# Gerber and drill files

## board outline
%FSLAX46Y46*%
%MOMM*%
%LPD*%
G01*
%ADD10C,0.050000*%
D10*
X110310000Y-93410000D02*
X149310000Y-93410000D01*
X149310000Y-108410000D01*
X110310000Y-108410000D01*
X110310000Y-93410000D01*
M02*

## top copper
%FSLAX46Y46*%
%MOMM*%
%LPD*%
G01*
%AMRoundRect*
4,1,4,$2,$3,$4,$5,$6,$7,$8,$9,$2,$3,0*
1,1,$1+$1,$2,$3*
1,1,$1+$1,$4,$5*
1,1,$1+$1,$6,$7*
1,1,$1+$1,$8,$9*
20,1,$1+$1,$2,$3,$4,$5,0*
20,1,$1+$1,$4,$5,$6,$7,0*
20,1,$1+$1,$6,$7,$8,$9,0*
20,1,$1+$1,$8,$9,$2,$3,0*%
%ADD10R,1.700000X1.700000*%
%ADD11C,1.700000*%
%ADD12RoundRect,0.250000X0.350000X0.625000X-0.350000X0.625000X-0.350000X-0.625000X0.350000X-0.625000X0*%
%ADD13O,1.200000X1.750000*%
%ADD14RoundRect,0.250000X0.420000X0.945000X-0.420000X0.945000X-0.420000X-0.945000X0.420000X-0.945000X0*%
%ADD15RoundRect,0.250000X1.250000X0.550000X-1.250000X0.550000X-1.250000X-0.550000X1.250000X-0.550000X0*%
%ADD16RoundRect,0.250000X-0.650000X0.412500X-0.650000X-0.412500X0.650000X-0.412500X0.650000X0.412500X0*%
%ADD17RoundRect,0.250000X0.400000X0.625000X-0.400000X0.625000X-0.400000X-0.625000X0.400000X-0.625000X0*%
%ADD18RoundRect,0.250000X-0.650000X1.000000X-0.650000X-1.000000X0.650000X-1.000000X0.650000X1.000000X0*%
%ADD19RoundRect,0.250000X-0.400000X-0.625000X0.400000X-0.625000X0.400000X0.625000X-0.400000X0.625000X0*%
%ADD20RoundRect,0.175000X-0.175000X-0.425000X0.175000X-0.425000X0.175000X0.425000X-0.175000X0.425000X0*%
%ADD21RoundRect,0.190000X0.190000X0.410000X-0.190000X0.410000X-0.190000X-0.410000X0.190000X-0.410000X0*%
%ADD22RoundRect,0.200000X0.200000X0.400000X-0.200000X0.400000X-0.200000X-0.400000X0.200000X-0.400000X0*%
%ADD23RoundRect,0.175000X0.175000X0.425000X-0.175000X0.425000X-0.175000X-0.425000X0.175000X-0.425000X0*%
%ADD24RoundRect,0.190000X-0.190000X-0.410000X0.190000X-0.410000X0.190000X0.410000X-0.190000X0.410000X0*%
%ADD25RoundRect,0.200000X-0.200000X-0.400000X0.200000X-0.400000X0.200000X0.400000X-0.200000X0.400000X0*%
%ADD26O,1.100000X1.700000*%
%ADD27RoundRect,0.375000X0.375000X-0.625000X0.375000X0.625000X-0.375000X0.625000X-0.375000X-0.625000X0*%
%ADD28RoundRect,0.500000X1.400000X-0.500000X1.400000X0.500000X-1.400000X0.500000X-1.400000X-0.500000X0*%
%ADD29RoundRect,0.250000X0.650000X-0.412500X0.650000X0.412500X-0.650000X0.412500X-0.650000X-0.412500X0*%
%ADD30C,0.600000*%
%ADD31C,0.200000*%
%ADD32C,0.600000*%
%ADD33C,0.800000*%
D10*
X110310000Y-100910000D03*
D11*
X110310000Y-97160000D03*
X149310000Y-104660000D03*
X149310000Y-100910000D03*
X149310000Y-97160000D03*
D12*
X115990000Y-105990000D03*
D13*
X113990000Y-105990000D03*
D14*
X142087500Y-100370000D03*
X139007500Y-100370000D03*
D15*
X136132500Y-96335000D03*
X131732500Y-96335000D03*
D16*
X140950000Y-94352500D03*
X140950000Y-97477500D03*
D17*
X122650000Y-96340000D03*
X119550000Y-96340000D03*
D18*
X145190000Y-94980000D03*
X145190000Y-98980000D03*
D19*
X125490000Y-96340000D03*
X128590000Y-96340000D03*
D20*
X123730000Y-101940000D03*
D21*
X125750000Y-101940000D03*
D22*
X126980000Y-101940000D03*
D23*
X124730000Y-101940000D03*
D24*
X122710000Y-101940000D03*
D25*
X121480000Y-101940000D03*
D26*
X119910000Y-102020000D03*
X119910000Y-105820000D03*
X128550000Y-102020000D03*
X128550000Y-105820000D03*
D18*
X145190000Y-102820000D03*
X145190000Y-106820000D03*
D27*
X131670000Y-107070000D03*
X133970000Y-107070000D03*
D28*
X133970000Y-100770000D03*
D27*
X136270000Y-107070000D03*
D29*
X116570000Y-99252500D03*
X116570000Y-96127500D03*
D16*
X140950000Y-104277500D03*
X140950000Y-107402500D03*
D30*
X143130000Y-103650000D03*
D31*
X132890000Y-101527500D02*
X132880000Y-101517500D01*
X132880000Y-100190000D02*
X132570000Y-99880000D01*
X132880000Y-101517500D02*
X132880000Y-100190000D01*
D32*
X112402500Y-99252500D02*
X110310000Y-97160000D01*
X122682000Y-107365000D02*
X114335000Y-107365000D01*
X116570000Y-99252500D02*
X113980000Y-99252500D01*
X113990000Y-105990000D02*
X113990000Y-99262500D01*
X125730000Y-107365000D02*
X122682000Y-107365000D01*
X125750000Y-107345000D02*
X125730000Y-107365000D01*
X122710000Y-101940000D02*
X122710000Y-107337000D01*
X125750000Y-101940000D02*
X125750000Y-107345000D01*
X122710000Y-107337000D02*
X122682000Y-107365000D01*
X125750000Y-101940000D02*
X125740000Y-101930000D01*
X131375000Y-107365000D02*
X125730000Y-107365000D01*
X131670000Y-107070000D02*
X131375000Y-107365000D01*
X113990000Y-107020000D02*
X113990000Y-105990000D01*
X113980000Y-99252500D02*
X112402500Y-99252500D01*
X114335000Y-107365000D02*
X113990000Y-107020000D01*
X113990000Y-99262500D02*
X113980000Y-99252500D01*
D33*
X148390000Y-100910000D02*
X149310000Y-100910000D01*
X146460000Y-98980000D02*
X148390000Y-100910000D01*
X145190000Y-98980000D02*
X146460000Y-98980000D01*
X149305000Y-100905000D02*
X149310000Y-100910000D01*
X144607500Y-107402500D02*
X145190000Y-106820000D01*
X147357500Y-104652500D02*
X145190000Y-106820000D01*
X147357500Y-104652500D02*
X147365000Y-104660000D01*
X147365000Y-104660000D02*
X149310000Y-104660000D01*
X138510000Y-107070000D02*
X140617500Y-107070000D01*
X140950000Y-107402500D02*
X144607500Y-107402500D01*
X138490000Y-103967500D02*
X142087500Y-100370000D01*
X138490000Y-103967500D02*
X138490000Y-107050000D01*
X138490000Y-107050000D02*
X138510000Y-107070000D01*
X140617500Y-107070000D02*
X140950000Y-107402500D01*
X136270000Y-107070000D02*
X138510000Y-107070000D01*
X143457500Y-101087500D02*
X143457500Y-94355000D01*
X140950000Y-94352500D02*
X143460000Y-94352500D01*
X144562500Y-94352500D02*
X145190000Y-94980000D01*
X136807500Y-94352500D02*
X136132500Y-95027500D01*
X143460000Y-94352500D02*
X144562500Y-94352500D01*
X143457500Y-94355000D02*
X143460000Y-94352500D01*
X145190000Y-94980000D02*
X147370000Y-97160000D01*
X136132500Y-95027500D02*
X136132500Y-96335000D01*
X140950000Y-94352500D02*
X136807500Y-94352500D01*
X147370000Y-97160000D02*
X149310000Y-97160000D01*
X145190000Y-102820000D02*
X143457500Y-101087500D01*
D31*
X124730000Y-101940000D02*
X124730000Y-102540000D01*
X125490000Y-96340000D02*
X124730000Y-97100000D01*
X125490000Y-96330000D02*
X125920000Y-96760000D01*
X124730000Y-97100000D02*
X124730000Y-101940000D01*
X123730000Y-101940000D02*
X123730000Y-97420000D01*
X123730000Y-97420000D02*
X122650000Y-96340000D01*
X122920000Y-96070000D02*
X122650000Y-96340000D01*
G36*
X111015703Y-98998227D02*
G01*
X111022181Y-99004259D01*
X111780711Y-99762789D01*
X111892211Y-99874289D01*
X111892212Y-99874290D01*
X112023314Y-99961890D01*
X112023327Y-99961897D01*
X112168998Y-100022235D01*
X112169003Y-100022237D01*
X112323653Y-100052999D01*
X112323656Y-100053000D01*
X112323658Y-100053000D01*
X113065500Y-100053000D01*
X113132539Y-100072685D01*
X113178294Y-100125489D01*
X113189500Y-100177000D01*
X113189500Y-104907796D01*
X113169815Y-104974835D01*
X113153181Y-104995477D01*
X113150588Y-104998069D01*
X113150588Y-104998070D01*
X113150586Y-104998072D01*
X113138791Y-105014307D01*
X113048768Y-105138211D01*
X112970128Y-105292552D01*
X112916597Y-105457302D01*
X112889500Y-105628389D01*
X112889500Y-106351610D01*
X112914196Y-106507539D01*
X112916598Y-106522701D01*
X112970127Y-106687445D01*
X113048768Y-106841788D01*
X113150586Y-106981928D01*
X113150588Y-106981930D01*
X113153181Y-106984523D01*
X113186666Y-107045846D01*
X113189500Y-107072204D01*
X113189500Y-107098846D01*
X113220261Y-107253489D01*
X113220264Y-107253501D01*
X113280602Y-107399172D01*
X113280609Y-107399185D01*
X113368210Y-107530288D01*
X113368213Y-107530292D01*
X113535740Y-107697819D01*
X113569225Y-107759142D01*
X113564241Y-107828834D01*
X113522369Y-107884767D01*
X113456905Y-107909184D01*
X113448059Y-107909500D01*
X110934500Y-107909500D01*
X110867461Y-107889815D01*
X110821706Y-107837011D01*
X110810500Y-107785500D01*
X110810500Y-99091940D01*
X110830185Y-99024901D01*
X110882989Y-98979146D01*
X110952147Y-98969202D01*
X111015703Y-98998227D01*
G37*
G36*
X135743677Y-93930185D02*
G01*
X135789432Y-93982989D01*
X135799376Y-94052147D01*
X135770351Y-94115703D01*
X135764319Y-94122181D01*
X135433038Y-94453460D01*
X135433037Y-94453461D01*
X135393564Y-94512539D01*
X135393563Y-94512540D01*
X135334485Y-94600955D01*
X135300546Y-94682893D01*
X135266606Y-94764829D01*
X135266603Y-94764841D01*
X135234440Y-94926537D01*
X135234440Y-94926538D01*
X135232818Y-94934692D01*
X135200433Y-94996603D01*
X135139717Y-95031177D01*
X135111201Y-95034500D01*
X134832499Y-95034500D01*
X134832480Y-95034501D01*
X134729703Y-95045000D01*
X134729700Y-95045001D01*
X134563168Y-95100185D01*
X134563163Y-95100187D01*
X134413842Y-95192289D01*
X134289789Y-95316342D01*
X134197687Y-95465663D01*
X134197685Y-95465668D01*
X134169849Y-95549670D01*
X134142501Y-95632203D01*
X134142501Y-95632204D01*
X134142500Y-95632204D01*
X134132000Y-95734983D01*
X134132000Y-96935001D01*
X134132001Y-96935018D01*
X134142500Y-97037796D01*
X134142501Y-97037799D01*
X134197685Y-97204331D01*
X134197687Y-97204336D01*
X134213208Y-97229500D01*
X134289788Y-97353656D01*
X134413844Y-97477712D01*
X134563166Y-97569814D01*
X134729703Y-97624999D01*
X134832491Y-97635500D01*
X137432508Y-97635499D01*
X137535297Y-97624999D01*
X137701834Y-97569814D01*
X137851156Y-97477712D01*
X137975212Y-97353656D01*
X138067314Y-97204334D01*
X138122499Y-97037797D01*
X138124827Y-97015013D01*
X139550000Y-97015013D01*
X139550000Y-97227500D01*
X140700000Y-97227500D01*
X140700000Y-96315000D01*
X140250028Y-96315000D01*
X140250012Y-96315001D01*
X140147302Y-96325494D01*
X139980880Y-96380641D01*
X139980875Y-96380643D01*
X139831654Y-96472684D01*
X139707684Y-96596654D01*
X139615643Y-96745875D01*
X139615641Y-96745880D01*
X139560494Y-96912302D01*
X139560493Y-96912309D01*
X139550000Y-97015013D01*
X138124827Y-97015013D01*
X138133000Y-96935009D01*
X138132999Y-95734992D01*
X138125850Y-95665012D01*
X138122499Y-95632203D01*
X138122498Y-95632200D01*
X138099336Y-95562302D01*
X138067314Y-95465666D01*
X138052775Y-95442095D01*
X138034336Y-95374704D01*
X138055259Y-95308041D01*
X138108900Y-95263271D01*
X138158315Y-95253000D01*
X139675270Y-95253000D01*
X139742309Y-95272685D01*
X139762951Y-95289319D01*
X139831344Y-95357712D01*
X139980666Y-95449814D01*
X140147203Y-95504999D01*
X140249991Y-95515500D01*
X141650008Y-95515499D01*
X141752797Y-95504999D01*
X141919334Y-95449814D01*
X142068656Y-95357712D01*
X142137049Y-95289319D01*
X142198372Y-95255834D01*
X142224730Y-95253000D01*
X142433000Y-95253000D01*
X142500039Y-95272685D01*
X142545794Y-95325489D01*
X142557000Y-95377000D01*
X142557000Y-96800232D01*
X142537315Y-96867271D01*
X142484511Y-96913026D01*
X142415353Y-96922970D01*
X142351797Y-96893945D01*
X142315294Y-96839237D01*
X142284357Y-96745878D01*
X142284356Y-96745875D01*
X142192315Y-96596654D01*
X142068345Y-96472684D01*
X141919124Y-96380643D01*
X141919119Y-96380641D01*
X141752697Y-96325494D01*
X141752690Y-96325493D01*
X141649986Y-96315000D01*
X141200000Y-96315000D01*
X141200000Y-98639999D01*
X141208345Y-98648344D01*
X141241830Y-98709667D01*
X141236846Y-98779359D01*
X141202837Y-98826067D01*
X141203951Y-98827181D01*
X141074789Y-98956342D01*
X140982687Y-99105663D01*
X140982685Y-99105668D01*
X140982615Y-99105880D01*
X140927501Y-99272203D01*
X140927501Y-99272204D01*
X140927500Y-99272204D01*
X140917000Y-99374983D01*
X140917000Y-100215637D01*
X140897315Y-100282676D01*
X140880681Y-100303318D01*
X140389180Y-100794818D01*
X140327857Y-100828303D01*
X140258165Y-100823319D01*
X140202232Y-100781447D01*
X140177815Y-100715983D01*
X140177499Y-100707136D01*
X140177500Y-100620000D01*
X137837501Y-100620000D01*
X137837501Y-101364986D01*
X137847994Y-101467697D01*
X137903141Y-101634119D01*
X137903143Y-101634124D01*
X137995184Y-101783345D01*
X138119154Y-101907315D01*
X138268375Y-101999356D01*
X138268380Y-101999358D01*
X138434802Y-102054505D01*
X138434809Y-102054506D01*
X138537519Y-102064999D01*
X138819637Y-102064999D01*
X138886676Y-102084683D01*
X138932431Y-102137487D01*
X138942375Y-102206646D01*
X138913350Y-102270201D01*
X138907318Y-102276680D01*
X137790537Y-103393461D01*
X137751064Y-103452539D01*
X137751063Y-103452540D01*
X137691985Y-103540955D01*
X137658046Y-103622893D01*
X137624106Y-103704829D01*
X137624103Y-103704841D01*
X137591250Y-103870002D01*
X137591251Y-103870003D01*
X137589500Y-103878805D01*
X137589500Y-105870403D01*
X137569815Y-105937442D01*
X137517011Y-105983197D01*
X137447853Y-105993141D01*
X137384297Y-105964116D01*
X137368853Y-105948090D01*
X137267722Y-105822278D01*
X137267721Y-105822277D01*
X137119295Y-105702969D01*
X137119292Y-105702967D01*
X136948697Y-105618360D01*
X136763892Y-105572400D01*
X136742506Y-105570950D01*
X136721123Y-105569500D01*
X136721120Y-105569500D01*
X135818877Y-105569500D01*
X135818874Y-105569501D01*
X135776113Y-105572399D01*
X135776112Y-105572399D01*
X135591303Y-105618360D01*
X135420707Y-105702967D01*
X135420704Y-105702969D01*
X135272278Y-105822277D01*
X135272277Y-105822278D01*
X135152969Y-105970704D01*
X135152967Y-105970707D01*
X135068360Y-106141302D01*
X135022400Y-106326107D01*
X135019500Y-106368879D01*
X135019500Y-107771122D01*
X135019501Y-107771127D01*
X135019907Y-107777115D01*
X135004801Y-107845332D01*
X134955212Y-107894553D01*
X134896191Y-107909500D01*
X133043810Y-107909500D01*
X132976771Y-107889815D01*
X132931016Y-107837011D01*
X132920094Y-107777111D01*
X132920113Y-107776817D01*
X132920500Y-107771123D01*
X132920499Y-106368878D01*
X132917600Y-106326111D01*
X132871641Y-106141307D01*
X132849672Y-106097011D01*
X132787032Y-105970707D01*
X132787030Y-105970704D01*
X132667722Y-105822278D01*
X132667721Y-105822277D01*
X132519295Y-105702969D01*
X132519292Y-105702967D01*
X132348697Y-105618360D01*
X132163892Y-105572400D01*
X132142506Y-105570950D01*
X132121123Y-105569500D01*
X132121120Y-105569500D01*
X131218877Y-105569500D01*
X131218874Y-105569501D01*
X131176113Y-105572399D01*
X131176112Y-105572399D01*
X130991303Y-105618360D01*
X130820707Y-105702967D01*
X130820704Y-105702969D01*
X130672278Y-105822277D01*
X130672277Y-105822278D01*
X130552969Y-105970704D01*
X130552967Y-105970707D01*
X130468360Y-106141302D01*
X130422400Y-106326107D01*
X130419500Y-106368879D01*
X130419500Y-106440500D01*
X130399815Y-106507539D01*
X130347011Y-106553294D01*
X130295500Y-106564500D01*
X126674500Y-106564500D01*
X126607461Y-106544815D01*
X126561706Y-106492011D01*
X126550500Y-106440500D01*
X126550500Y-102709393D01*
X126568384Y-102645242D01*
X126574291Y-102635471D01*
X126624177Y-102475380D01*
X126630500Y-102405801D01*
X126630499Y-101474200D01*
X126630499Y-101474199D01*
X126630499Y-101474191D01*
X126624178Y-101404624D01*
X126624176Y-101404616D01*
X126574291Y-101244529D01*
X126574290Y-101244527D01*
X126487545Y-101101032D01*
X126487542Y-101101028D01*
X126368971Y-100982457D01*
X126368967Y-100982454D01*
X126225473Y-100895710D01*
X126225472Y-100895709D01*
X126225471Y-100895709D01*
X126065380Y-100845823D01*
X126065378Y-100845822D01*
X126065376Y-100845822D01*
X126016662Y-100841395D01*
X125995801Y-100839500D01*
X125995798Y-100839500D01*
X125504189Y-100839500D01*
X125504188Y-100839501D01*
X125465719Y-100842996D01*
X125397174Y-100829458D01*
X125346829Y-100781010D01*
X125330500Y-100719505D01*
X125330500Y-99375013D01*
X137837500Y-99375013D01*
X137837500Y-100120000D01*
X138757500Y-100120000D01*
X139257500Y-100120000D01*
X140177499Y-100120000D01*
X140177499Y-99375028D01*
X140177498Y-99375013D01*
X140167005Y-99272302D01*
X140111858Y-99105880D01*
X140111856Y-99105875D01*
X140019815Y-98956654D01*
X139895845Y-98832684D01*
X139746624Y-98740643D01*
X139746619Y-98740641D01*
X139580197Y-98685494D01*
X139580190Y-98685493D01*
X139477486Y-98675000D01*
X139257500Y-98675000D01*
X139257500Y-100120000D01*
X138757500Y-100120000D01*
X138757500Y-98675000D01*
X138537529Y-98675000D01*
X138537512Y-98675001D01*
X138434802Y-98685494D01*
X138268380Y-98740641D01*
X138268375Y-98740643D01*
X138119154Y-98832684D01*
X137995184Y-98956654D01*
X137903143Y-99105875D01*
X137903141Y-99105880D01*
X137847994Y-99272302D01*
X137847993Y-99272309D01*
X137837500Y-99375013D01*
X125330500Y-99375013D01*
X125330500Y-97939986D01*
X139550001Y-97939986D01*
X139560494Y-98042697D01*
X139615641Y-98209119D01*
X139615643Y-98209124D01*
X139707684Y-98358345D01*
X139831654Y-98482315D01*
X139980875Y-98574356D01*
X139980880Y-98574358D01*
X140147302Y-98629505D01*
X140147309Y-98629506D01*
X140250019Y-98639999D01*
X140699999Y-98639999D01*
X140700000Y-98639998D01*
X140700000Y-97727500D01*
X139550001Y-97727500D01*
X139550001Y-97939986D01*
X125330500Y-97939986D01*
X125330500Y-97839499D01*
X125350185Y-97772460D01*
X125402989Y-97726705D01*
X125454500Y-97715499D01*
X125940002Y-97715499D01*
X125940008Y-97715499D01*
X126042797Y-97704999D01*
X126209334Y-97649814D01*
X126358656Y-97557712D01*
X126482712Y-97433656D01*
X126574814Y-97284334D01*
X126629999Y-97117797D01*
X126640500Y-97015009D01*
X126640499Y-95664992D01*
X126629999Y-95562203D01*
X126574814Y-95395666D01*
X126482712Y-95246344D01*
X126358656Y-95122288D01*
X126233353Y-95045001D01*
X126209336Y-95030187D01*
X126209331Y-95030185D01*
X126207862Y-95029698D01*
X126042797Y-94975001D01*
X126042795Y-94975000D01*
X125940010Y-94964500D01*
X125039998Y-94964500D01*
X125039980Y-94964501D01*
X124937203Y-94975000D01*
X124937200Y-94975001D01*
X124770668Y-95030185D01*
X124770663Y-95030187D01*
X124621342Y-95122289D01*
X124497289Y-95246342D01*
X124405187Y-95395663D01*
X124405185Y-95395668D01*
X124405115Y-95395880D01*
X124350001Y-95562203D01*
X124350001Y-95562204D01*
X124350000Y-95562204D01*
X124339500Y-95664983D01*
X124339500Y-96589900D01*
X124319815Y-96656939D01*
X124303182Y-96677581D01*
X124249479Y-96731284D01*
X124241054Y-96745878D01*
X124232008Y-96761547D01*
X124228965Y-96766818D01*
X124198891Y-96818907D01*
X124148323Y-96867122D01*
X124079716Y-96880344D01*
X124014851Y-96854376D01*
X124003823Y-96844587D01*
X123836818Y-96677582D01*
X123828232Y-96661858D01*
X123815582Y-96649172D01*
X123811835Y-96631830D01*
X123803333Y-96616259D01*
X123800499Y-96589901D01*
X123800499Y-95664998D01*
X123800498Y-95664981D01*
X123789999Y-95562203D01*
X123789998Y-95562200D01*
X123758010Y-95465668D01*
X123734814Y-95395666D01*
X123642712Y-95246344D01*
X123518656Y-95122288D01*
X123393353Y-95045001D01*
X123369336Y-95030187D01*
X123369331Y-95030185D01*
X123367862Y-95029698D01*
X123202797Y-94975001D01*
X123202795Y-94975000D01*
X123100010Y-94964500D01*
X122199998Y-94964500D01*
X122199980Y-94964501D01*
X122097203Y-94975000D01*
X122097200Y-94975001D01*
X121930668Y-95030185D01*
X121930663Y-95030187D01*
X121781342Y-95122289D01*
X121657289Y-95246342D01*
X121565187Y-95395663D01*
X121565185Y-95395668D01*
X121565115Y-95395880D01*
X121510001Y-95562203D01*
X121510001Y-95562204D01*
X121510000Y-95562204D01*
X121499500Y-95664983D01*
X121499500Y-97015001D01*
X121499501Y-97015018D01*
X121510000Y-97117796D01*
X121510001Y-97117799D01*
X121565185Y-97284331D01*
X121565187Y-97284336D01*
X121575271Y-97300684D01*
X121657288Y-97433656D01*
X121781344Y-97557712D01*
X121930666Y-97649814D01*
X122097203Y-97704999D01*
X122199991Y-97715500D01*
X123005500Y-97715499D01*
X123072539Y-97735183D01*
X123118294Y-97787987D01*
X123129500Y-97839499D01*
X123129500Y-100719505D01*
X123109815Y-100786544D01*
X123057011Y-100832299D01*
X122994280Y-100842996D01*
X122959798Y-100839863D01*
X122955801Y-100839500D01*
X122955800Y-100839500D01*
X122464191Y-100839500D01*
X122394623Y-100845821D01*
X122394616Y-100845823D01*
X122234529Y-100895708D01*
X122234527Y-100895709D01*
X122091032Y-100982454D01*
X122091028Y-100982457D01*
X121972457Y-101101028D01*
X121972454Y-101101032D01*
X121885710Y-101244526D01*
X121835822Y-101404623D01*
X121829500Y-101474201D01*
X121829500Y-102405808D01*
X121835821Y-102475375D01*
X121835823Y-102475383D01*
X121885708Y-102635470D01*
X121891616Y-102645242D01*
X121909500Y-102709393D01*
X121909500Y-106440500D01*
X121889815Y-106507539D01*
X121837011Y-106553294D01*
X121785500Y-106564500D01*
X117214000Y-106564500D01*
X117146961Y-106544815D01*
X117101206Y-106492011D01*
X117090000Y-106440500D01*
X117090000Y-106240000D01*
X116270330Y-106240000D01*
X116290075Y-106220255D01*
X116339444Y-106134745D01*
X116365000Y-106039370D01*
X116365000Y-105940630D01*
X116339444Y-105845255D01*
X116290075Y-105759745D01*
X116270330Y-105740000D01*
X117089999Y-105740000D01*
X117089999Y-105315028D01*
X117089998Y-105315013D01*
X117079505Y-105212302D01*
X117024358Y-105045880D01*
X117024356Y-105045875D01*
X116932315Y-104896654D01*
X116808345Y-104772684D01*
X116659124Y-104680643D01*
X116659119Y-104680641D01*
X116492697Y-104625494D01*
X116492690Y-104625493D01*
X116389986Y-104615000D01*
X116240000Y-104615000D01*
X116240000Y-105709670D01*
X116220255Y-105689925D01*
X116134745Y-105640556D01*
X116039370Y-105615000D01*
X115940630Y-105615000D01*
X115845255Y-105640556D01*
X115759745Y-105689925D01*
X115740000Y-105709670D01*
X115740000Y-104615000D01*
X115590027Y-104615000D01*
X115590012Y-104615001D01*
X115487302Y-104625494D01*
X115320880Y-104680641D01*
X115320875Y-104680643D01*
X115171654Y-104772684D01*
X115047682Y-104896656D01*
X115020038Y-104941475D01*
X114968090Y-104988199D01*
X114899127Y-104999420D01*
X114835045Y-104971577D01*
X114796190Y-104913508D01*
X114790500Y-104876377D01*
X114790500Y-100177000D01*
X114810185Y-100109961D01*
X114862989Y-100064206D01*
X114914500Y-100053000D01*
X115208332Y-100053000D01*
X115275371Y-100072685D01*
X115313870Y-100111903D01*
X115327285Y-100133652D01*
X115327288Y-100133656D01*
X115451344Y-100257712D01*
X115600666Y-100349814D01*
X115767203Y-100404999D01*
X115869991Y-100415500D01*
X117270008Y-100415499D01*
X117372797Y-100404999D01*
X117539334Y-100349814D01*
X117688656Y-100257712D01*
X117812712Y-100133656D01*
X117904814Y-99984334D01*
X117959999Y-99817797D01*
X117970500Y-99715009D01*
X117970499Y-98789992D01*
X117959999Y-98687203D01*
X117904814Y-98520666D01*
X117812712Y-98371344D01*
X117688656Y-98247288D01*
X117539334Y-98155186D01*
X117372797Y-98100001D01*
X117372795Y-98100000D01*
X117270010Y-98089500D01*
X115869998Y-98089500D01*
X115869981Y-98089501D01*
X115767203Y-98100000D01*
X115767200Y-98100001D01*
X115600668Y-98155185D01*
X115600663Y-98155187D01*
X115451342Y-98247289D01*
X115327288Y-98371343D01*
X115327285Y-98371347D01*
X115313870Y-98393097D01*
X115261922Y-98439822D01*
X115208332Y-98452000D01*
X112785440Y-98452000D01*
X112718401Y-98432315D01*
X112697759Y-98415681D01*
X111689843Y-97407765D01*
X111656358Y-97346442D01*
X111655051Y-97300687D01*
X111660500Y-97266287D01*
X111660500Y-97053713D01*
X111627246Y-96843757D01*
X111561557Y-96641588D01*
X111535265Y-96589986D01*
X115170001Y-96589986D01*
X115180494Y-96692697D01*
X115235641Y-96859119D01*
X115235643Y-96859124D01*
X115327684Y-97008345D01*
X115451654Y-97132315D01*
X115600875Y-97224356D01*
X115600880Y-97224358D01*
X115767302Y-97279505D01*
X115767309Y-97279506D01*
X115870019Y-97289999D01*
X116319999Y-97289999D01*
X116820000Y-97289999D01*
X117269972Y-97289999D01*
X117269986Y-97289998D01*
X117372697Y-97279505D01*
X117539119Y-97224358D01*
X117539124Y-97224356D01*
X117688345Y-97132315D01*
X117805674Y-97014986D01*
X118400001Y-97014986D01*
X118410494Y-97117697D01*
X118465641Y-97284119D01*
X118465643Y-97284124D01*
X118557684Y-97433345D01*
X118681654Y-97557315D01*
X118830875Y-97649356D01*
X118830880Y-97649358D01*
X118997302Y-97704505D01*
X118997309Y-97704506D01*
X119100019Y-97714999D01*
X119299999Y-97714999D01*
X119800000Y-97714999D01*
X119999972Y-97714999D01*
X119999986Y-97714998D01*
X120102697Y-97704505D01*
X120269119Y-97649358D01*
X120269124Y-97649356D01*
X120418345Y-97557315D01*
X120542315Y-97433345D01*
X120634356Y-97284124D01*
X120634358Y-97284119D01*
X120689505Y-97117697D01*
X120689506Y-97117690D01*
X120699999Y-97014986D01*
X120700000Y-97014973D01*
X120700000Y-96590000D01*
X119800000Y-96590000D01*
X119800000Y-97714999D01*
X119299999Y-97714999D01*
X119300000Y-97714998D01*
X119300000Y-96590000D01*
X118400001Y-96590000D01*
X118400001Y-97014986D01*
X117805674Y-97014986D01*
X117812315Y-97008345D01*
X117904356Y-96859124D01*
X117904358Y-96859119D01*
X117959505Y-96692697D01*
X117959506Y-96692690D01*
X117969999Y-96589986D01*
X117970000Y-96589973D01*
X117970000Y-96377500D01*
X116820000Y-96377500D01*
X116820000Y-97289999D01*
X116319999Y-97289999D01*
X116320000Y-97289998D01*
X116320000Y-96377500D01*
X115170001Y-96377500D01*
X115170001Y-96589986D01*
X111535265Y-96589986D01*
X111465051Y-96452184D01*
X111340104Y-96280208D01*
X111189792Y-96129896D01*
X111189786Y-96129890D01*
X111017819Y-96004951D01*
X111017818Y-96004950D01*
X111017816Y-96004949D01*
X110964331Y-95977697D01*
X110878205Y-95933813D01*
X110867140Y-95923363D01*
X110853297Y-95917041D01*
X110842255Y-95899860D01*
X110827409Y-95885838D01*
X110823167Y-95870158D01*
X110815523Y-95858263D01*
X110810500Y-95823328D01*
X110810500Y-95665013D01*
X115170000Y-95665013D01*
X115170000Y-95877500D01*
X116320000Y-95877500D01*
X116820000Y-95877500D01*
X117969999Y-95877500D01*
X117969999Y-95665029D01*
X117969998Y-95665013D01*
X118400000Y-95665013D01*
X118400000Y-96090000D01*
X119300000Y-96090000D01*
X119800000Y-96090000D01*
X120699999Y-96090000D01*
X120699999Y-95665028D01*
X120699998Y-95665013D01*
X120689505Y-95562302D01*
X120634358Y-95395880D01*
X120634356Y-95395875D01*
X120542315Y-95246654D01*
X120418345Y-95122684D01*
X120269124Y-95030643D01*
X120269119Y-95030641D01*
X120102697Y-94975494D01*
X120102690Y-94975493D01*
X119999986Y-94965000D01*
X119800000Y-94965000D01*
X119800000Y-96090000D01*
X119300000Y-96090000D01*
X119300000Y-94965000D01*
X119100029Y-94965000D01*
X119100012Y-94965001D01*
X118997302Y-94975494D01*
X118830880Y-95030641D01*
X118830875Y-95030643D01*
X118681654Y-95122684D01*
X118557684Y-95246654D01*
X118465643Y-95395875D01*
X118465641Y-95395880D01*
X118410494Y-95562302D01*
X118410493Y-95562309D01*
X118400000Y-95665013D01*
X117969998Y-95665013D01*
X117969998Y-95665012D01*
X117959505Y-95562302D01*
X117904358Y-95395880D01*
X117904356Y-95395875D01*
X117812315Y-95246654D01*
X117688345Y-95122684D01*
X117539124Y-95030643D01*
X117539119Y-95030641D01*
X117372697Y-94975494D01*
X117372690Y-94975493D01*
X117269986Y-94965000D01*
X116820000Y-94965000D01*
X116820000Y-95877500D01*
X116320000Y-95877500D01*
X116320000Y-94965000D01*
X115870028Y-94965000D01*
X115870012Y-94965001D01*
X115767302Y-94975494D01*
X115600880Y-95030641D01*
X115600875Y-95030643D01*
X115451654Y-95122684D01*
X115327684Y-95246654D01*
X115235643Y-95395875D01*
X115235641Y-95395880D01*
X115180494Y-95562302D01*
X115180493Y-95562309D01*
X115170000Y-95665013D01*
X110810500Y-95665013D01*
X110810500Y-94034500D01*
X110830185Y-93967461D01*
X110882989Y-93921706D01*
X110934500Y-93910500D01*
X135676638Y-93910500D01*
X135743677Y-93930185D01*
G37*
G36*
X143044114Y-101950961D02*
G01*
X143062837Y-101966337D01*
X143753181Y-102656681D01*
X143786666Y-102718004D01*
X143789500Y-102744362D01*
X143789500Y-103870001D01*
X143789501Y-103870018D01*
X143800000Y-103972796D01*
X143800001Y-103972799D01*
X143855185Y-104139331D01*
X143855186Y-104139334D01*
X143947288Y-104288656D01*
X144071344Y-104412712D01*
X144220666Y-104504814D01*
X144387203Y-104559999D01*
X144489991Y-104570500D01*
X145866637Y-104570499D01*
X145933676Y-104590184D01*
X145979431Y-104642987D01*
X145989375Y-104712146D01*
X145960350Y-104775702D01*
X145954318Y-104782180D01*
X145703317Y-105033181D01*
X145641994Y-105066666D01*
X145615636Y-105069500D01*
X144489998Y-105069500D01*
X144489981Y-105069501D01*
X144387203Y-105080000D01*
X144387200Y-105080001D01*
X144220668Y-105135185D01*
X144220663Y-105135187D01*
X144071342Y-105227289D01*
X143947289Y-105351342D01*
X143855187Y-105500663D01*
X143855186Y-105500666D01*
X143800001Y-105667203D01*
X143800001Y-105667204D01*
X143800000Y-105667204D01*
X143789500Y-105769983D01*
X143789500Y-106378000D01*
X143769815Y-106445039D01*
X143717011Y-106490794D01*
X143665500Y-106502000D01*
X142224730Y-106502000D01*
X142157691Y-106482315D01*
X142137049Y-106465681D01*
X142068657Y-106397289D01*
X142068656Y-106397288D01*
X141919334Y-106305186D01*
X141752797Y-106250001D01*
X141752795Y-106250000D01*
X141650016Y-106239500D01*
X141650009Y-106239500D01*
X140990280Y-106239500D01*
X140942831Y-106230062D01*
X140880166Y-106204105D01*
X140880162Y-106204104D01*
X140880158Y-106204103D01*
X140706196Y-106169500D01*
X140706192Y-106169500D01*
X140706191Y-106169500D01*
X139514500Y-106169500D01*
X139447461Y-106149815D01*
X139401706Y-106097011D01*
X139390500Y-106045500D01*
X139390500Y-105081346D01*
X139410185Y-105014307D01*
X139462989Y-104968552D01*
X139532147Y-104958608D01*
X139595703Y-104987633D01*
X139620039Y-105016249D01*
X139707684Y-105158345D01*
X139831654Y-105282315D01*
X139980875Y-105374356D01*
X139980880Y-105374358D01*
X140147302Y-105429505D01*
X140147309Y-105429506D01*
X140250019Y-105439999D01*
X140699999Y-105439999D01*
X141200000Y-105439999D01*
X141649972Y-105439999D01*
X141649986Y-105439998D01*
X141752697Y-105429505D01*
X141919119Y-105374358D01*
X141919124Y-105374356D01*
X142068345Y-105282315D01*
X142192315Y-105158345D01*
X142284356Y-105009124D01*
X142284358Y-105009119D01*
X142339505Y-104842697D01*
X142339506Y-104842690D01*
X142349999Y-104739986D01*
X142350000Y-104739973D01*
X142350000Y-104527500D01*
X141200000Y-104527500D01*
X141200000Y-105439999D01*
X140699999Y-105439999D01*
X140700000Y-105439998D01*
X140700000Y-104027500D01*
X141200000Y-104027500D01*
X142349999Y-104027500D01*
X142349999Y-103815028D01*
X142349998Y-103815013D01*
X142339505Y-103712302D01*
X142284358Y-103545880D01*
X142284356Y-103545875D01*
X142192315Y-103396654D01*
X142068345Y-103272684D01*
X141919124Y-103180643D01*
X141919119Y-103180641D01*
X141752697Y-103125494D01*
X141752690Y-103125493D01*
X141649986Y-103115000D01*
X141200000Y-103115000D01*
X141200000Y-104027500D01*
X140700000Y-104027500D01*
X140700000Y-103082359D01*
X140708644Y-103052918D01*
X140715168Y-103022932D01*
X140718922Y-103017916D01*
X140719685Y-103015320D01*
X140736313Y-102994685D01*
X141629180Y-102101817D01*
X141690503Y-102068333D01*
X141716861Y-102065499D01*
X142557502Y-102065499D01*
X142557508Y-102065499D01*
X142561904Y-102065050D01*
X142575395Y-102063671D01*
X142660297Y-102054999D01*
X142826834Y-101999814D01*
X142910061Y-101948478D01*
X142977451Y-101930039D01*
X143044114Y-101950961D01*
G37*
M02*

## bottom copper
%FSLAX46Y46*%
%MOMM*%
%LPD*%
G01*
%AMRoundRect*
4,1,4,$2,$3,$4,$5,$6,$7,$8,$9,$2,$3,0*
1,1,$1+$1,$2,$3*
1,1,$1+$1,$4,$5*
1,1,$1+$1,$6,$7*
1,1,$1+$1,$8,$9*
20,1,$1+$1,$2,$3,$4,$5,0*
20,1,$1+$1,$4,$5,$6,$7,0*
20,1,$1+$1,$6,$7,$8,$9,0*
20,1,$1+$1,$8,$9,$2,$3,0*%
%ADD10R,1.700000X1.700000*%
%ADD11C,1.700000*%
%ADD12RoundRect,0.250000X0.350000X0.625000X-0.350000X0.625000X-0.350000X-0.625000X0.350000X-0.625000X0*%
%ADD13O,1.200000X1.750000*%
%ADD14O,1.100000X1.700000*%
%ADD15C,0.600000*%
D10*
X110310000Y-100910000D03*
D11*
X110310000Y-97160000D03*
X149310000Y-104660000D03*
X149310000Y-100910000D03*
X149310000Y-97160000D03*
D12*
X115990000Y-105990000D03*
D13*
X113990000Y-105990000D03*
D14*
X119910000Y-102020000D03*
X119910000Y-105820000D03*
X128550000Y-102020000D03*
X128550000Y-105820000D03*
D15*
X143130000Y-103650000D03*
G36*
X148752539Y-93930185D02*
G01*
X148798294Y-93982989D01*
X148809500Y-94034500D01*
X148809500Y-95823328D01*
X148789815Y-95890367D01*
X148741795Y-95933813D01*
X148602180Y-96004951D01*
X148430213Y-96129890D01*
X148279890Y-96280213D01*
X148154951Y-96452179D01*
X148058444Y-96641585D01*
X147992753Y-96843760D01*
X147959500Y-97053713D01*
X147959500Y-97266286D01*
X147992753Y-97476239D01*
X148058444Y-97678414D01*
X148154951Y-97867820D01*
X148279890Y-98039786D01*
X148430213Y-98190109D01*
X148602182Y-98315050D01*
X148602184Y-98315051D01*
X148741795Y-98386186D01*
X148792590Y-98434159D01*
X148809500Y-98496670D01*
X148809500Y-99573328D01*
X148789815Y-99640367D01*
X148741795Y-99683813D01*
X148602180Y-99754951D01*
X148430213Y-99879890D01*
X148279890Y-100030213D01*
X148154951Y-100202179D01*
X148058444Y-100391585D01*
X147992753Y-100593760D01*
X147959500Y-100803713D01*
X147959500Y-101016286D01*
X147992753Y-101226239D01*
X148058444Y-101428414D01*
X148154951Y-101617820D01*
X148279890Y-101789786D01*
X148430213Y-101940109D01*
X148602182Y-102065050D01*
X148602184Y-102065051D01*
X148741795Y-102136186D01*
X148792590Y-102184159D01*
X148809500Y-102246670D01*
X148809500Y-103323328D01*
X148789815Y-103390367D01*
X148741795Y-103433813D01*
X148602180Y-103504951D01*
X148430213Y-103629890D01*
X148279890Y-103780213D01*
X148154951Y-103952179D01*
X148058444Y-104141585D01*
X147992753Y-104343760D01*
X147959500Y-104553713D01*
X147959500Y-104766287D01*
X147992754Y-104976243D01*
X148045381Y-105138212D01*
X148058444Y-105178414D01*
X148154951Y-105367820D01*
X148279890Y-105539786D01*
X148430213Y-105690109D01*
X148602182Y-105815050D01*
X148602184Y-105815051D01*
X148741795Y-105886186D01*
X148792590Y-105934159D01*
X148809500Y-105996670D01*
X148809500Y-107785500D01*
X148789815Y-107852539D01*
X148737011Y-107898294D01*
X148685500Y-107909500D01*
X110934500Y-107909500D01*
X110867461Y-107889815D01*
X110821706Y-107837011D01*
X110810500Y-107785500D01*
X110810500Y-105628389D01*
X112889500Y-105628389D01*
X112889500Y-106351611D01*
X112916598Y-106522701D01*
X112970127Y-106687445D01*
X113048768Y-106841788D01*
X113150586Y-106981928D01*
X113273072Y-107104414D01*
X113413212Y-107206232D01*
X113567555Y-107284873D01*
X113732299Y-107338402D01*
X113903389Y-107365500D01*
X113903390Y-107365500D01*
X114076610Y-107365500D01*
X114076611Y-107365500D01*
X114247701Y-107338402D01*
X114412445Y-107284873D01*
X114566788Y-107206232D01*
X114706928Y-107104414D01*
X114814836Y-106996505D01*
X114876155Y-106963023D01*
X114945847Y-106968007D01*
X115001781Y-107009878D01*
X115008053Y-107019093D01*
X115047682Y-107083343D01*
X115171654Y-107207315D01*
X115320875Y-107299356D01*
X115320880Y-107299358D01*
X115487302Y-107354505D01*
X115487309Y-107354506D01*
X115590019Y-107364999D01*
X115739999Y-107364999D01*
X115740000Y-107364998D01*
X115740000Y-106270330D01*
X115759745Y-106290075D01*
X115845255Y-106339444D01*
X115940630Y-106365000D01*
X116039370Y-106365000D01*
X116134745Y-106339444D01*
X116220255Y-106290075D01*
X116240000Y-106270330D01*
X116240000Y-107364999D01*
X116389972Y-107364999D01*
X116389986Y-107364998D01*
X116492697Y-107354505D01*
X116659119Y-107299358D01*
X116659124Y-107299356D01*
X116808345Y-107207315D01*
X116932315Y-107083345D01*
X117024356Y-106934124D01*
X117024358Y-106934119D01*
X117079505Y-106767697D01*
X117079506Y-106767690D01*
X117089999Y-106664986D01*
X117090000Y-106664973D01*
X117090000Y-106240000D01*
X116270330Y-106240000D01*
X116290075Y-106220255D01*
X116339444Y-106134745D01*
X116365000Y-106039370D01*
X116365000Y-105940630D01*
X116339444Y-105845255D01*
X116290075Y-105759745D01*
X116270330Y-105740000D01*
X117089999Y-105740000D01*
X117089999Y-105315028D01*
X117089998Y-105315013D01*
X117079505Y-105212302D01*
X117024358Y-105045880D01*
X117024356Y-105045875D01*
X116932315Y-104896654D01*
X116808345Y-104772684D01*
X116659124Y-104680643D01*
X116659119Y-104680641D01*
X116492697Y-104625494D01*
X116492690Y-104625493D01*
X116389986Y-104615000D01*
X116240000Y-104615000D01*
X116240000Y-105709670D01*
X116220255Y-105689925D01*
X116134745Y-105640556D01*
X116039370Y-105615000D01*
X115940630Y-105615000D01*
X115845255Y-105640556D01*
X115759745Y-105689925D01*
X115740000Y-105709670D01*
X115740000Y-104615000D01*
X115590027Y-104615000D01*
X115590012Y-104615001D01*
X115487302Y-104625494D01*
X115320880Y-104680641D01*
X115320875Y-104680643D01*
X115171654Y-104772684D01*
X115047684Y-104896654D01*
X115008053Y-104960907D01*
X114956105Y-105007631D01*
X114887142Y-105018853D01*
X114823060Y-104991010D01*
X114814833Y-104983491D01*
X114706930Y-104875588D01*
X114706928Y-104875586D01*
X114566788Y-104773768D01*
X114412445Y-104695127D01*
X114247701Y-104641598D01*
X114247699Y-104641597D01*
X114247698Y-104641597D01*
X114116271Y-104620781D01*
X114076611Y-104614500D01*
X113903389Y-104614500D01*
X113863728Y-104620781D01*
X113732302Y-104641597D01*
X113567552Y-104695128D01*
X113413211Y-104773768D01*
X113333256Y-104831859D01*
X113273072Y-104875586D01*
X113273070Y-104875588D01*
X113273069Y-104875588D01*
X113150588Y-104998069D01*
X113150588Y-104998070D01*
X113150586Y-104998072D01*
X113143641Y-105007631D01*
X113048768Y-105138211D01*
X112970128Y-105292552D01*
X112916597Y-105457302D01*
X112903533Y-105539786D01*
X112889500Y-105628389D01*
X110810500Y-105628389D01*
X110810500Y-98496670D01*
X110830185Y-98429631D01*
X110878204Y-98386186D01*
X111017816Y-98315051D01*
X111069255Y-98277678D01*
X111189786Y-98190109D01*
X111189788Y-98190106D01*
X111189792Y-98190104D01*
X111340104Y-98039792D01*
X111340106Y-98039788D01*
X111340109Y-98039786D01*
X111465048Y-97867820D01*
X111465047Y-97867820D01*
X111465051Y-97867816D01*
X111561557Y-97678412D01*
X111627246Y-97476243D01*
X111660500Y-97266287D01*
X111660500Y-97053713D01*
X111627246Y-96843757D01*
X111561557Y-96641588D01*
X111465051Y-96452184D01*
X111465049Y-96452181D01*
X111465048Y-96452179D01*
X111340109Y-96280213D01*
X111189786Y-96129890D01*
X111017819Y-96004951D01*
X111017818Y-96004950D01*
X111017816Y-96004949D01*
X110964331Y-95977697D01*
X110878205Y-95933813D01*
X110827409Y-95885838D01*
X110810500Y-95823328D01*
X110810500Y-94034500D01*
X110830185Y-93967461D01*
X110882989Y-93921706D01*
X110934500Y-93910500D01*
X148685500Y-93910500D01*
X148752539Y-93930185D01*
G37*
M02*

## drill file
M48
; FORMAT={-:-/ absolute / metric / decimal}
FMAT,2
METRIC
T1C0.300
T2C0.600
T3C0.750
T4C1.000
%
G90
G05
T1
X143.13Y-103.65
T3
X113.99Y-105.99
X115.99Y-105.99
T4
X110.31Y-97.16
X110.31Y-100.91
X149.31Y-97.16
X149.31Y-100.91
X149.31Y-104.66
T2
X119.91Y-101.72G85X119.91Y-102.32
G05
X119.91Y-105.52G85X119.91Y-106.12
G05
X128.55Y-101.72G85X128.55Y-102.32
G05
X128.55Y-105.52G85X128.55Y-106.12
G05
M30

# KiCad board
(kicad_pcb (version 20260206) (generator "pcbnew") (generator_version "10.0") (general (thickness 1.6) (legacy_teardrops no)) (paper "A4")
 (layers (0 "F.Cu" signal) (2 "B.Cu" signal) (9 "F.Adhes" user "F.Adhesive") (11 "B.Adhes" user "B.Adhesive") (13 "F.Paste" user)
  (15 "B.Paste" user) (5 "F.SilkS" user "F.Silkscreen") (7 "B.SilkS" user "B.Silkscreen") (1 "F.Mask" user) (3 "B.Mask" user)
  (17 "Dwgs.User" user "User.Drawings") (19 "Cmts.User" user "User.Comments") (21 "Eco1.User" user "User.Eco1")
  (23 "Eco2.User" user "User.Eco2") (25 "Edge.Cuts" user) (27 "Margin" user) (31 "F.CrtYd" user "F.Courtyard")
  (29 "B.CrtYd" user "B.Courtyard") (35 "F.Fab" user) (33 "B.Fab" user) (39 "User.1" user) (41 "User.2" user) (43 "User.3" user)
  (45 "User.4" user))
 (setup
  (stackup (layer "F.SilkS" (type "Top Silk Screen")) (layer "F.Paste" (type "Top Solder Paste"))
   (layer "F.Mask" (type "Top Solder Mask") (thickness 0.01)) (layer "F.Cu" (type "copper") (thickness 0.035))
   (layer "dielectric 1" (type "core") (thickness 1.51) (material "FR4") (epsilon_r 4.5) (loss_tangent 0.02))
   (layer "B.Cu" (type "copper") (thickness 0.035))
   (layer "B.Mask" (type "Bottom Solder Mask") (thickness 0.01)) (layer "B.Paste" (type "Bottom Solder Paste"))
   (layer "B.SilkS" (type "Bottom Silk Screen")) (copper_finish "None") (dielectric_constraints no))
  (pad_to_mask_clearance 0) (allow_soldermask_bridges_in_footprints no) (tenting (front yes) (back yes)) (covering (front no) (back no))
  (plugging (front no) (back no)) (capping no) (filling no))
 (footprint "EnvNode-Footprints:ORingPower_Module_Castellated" (layer "F.Cu") (at 129.81 100.91)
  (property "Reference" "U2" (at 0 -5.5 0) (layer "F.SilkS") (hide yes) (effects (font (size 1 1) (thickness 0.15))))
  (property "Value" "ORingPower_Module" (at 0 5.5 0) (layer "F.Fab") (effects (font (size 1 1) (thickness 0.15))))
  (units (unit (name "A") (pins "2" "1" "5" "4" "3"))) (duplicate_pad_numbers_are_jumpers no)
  (pad "1" thru_hole rect (at -19.5 0) (size 1.7 1.7) (drill 1) (layers "*.Cu" "*.Mask") (remove_unused_layers no) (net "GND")
   (zone_connect 2))
  (pad "2" thru_hole circle (at -19.5 -3.75) (size 1.7 1.7) (drill 1) (layers "*.Cu" "*.Mask") (remove_unused_layers no) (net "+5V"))
  (pad "3" thru_hole circle (at 19.5 3.75) (size 1.7 1.7) (drill 1) (layers "*.Cu" "*.Mask") (remove_unused_layers no) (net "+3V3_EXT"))
  (pad "4" thru_hole circle (at 19.5 0) (size 1.7 1.7) (drill 1) (layers "*.Cu" "*.Mask") (remove_unused_layers no) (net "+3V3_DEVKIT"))
  (pad "5" thru_hole circle (at 19.5 -3.75) (size 1.7 1.7) (drill 1) (layers "*.Cu" "*.Mask") (remove_unused_layers no) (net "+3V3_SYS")))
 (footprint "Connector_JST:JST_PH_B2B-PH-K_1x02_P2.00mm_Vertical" (layer "F.Cu") (at 115.99 105.99 180)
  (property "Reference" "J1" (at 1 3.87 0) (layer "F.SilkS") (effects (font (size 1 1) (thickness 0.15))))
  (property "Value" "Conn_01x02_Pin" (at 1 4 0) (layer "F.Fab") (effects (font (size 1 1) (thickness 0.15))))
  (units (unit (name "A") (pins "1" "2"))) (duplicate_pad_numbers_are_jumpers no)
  (pad "1" thru_hole roundrect (at 0 0 180) (size 1.2 1.75) (drill 0.75) (layers "*.Cu" "*.Mask") (remove_unused_layers no)
   (roundrect_rratio 0.208333) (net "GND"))
  (pad "2" thru_hole oval (at 2 0 180) (size 1.2 1.75) (drill 0.75) (layers "*.Cu" "*.Mask") (remove_unused_layers no) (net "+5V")
   (zone_connect 2)))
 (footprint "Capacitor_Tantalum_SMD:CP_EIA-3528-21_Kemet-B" (layer "F.Cu") (at 140.5475 100.37 180)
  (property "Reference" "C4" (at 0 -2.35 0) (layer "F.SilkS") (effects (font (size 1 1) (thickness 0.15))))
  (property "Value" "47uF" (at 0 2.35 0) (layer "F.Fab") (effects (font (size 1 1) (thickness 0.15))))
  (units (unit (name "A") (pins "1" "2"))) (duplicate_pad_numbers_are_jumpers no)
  (pad "1" smd roundrect (at -1.54 0 180) (size 1.34 2.39) (layers "F.Cu" "F.Mask" "F.Paste") (roundrect_rratio 0.186567) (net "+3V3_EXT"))
  (pad "2" smd roundrect (at 1.54 0 180) (size 1.34 2.39) (layers "F.Cu" "F.Mask" "F.Paste") (roundrect_rratio 0.186567) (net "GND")))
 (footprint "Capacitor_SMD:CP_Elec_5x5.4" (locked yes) (layer "F.Cu") (at 133.9325 96.335 180)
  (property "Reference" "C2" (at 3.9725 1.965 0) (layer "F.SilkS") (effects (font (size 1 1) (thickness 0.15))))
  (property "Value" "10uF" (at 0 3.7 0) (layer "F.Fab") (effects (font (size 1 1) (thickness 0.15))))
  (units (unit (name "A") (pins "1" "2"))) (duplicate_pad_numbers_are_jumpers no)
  (pad "1" smd roundrect (at -2.2 0 180) (size 3 1.6) (layers "F.Cu" "F.Mask" "F.Paste") (roundrect_rratio 0.15625) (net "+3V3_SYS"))
  (pad "2" smd roundrect (at 2.2 0 180) (size 3 1.6) (layers "F.Cu" "F.Mask" "F.Paste") (roundrect_rratio 0.15625) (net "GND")
   (zone_connect 2)))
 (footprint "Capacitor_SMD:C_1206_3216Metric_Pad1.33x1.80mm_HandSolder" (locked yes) (layer "F.Cu") (at 140.95 95.915 -90)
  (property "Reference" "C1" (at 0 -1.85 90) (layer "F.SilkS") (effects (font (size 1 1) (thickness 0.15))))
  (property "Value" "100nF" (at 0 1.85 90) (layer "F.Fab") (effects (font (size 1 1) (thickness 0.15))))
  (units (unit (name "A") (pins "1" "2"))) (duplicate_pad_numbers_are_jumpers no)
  (pad "1" smd roundrect (at -1.5625 0 270) (size 1.325 1.8) (layers "F.Cu" "F.Mask" "F.Paste") (roundrect_rratio 0.188679) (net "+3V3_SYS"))
  (pad "2" smd roundrect (at 1.5625 0 270) (size 1.325 1.8) (layers "F.Cu" "F.Mask" "F.Paste") (roundrect_rratio 0.188679) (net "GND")))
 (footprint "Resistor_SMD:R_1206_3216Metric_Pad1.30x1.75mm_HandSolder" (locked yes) (layer "F.Cu") (at 121.1 96.34 180)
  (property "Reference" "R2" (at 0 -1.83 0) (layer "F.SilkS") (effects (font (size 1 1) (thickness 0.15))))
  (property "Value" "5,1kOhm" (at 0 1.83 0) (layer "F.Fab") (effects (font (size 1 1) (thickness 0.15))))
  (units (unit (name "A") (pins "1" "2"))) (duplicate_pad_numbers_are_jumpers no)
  (pad "1" smd roundrect (at -1.55 0 180) (size 1.3 1.75) (layers "F.Cu" "F.Mask" "F.Paste") (roundrect_rratio 0.192308)
   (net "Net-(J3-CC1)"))
  (pad "2" smd roundrect (at 1.55 0 180) (size 1.3 1.75) (layers "F.Cu" "F.Mask" "F.Paste") (roundrect_rratio 0.192308) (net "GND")))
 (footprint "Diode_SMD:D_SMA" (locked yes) (layer "F.Cu") (at 145.19 96.98 -90)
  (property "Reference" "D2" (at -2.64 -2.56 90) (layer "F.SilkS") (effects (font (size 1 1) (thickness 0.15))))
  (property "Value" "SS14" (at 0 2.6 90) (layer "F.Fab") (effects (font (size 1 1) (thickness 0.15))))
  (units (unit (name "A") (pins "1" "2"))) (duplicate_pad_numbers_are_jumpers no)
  (pad "1" smd roundrect (at -2 0 270) (size 2.5 1.8) (layers "F.Cu" "F.Mask" "F.Paste") (roundrect_rratio 0.1388888889) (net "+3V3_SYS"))
  (pad "2" smd roundrect (at 2 0 270) (size 2.5 1.8) (layers "F.Cu" "F.Mask" "F.Paste") (roundrect_rratio 0.1388888889) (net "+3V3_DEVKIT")))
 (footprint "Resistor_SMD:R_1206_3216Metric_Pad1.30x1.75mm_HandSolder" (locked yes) (layer "F.Cu") (at 127.04 96.34)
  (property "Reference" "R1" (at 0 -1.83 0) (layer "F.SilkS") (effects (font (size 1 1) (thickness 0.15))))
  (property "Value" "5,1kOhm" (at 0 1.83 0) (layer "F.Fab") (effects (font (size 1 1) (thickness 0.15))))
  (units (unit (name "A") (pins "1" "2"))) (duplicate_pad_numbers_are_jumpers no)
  (pad "1" smd roundrect (at -1.55 0) (size 1.3 1.75) (layers "F.Cu" "F.Mask" "F.Paste") (roundrect_rratio 0.192308) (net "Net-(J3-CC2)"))
  (pad "2" smd roundrect (at 1.55 0) (size 1.3 1.75) (layers "F.Cu" "F.Mask" "F.Paste") (roundrect_rratio 0.192308) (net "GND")
   (zone_connect 2)))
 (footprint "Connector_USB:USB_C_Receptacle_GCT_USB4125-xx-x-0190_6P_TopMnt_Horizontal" (layer "F.Cu") (at 124.23 105.02)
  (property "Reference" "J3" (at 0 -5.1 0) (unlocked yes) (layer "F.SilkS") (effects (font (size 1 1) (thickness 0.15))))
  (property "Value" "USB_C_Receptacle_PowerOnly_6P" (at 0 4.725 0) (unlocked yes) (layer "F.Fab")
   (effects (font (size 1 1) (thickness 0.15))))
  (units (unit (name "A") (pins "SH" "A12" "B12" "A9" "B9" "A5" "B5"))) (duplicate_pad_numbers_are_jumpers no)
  (pad "A5" smd roundrect (at -0.5 -3.08) (size 0.7 1.2) (layers "F.Cu" "F.Mask" "F.Paste") (roundrect_rratio 0.25) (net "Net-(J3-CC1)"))
  (pad "A9" smd roundrect (at 1.52 -3.08 180) (size 0.76 1.2) (layers "F.Cu" "F.Mask" "F.Paste") (roundrect_rratio 0.25) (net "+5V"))
  (pad "A12" smd roundrect (at 2.75 -3.08 180) (size 0.8 1.2) (layers "F.Cu" "F.Mask" "F.Paste") (roundrect_rratio 0.25) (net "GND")
   (zone_connect 2))
  (pad "B5" smd roundrect (at 0.5 -3.08 180) (size 0.7 1.2) (layers "F.Cu" "F.Mask" "F.Paste") (roundrect_rratio 0.25) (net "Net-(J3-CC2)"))
  (pad "B9" smd roundrect (at -1.52 -3.08) (size 0.76 1.2) (layers "F.Cu" "F.Mask" "F.Paste") (roundrect_rratio 0.25) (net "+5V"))
  (pad "B12" smd roundrect (at -2.75 -3.08) (size 0.8 1.2) (layers "F.Cu" "F.Mask" "F.Paste") (roundrect_rratio 0.25) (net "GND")
   (zone_connect 2))
  (pad "SH" thru_hole oval (at -4.32 -3) (size 1.1 1.7) (drill oval 0.6 1.2) (layers "*.Cu" "*.Mask" "F.Paste") (remove_unused_layers no)
   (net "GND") (zone_connect 2))
  (pad "SH" thru_hole oval (at -4.32 0.8) (size 1.1 1.7) (drill oval 0.6 1.2) (layers "*.Cu" "*.Mask" "F.Paste") (remove_unused_layers no)
   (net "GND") (zone_connect 2))
  (pad "SH" thru_hole oval (at 4.32 -3) (size 1.1 1.7) (drill oval 0.6 1.2) (layers "*.Cu" "*.Mask" "F.Paste") (remove_unused_layers no)
   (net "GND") (zone_connect 2))
  (pad "SH" thru_hole oval (at 4.32 0.8) (size 1.1 1.7) (drill oval 0.6 1.2) (layers "*.Cu" "*.Mask" "F.Paste") (remove_unused_layers no)
   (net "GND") (zone_connect 2)))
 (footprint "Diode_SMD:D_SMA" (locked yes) (layer "F.Cu") (at 145.19 104.82 -90)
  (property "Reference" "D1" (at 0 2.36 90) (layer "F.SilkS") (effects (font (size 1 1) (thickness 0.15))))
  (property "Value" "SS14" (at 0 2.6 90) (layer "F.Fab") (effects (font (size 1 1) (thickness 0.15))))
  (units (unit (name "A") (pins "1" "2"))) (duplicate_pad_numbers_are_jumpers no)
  (pad "1" smd roundrect (at -2 0 270) (size 2.5 1.8) (layers "F.Cu" "F.Mask" "F.Paste") (roundrect_rratio 0.1388888889) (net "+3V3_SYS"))
  (pad "2" smd roundrect (at 2 0 270) (size 2.5 1.8) (layers "F.Cu" "F.Mask" "F.Paste") (roundrect_rratio 0.1388888889) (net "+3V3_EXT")))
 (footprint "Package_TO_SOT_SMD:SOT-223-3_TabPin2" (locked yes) (layer "F.Cu") (at 133.97 103.92 90)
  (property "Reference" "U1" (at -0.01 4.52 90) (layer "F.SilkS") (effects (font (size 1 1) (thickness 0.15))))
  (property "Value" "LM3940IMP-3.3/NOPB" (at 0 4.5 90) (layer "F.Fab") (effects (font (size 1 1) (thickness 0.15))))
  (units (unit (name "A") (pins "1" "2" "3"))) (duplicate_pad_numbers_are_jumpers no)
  (pad "1" smd roundrect (at -3.15 -2.3 90) (size 2 1.5) (layers "F.Cu" "F.Mask" "F.Paste") (roundrect_rratio 0.25) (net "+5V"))
  (pad "2" smd roundrect (at -3.15 0 90) (size 2 1.5) (layers "F.Cu" "F.Mask" "F.Paste") (roundrect_rratio 0.25) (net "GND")
   (zone_connect 2))
  (pad "2" smd roundrect (at 3.15 0 90) (size 2 3.8) (layers "F.Cu" "F.Mask" "F.Paste") (roundrect_rratio 0.25) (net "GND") (zone_connect 2))
  (pad "3" smd roundrect (at -3.15 2.3 90) (size 2 1.5) (layers "F.Cu" "F.Mask" "F.Paste") (roundrect_rratio 0.25) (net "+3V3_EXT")))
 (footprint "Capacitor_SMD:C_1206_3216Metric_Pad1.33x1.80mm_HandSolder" (layer "F.Cu") (at 116.57 97.69 90)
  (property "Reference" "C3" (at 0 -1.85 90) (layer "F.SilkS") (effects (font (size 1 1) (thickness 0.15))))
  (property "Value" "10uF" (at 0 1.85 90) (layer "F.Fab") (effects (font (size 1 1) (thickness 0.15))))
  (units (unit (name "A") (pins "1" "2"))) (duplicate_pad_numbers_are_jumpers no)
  (pad "1" smd roundrect (at -1.5625 0 90) (size 1.325 1.8) (layers "F.Cu" "F.Mask" "F.Paste") (roundrect_rratio 0.188679) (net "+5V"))
  (pad "2" smd roundrect (at 1.5625 0 90) (size 1.325 1.8) (layers "F.Cu" "F.Mask" "F.Paste") (roundrect_rratio 0.188679) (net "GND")))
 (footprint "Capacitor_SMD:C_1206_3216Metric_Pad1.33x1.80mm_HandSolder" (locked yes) (layer "F.Cu") (at 140.95 105.84 -90)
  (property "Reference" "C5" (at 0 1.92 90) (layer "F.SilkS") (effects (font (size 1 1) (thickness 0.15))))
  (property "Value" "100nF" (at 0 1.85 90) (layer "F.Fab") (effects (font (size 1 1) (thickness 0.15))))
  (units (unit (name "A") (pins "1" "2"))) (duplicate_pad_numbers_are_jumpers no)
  (pad "1" smd roundrect (at -1.5625 0 270) (size 1.325 1.8) (layers "F.Cu" "F.Mask" "F.Paste") (roundrect_rratio 0.188679) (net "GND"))
  (pad "2" smd roundrect (at 1.5625 0 270) (size 1.325 1.8) (layers "F.Cu" "F.Mask" "F.Paste") (roundrect_rratio 0.188679) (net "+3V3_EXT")))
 (gr_rect (start 110.31 93.41) (end 149.31 108.41) (stroke (width 0.05) (type solid)) (fill no) (locked yes) (layer "Edge.Cuts"))
 (segment (start 132.89 101.5275) (end 132.88 101.5175) (width 0.2) (layer "F.Cu") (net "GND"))
 (segment (start 132.88 100.19) (end 132.57 99.88) (width 0.2) (layer "F.Cu") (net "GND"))
 (segment (start 132.88 101.5175) (end 132.88 100.19) (width 0.2) (layer "F.Cu") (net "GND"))
 (via (at 143.13 103.65) (size 0.6) (drill 0.3) (layers "F.Cu" "B.Cu") (free yes) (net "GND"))
 (segment (start 112.4025 99.2525) (end 110.31 97.16) (width 0.6) (layer "F.Cu") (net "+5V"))
 (segment (start 122.682 107.365) (end 114.335 107.365) (width 0.6) (layer "F.Cu") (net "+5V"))
 (segment (start 116.57 99.2525) (end 113.98 99.2525) (width 0.6) (layer "F.Cu") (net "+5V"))
 (segment (start 113.99 105.99) (end 113.99 99.2625) (width 0.6) (layer "F.Cu") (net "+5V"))
 (segment (start 125.73 107.365) (end 122.682 107.365) (width 0.6) (layer "F.Cu") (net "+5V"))
 (segment (start 125.75 107.345) (end 125.73 107.365) (width 0.6) (layer "F.Cu") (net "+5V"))
 (segment (start 122.71 101.94) (end 122.71 107.337) (width 0.6) (layer "F.Cu") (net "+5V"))
 (segment (start 125.75 101.94) (end 125.75 107.345) (width 0.6) (layer "F.Cu") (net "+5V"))
 (segment (start 122.71 107.337) (end 122.682 107.365) (width 0.6) (layer "F.Cu") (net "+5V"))
 (segment (start 125.75 101.94) (end 125.74 101.93) (width 0.6) (layer "F.Cu") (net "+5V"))
 (segment (start 131.375 107.365) (end 125.73 107.365) (width 0.6) (layer "F.Cu") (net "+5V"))
 (segment (start 131.67 107.07) (end 131.375 107.365) (width 0.6) (layer "F.Cu") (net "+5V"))
 (segment (start 113.99 107.02) (end 113.99 105.99) (width 0.6) (layer "F.Cu") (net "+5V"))
 (segment (start 113.98 99.2525) (end 112.4025 99.2525) (width 0.6) (layer "F.Cu") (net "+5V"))
 (segment (start 114.335 107.365) (end 113.99 107.02) (width 0.6) (layer "F.Cu") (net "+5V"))
 (segment (start 113.99 99.2625) (end 113.98 99.2525) (width 0.6) (layer "F.Cu") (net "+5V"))
 (segment (start 148.39 100.91) (end 149.31 100.91) (width 0.8) (layer "F.Cu") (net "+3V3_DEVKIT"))
 (segment (start 146.46 98.98) (end 148.39 100.91) (width 0.8) (layer "F.Cu") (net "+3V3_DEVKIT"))
 (segment (start 145.19 98.98) (end 146.46 98.98) (width 0.8) (layer "F.Cu") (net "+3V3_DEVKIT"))
 (segment (start 149.305 100.905) (end 149.31 100.91) (width 0.8) (layer "F.Cu") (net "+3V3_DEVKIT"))
 (segment (start 144.6075 107.4025) (end 145.19 106.82) (width 0.8) (layer "F.Cu") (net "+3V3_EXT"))
 (segment (start 147.3575 104.6525) (end 145.19 106.82) (width 0.8) (layer "F.Cu") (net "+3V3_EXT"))
 (segment (start 147.3575 104.6525) (end 147.365 104.66) (width 0.8) (layer "F.Cu") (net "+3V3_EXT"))
 (segment (start 147.365 104.66) (end 149.31 104.66) (width 0.8) (layer "F.Cu") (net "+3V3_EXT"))
 (segment (start 138.51 107.07) (end 140.6175 107.07) (width 0.8) (layer "F.Cu") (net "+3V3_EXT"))
 (segment (start 140.95 107.4025) (end 144.6075 107.4025) (width 0.8) (layer "F.Cu") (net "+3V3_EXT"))
 (segment (start 138.49 103.9675) (end 142.0875 100.37) (width 0.8) (layer "F.Cu") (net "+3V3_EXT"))
 (segment (start 138.49 103.9675) (end 138.49 107.05) (width 0.8) (layer "F.Cu") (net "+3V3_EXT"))
 (segment (start 138.49 107.05) (end 138.51 107.07) (width 0.8) (layer "F.Cu") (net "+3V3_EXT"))
 (segment (start 140.6175 107.07) (end 140.95 107.4025) (width 0.8) (layer "F.Cu") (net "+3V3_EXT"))
 (segment (start 136.27 107.07) (end 138.51 107.07) (width 0.8) (layer "F.Cu") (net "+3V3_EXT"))
 (segment (start 143.4575 101.0875) (end 143.4575 94.355) (width 0.8) (layer "F.Cu") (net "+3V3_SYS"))
 (segment (start 140.95 94.3525) (end 143.46 94.3525) (width 0.8) (layer "F.Cu") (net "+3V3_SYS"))
 (segment (start 144.5625 94.3525) (end 145.19 94.98) (width 0.8) (layer "F.Cu") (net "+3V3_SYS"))
 (segment (start 136.8075 94.3525) (end 136.1325 95.0275) (width 0.8) (layer "F.Cu") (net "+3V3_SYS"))
 (segment (start 143.46 94.3525) (end 144.5625 94.3525) (width 0.8) (layer "F.Cu") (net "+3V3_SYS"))
 (segment (start 143.4575 94.355) (end 143.46 94.3525) (width 0.8) (layer "F.Cu") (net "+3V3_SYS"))
 (segment (start 145.19 94.98) (end 147.37 97.16) (width 0.8) (layer "F.Cu") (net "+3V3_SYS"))
 (segment (start 136.1325 95.0275) (end 136.1325 96.335) (width 0.8) (layer "F.Cu") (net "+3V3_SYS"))
 (segment (start 140.95 94.3525) (end 136.8075 94.3525) (width 0.8) (layer "F.Cu") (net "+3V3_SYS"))
 (segment (start 147.37 97.16) (end 149.31 97.16) (width 0.8) (layer "F.Cu") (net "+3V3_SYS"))
 (segment (start 145.19 102.82) (end 143.4575 101.0875) (width 0.8) (layer "F.Cu") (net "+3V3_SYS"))
 (segment (start 124.73 101.94) (end 124.73 102.54) (width 0.2) (layer "F.Cu") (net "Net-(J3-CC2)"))
 (segment (start 125.49 96.34) (end 124.73 97.1) (width 0.2) (layer "F.Cu") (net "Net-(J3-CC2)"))
 (segment (start 125.49 96.33) (end 125.92 96.76) (width 0.2) (layer "F.Cu") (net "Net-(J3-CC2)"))
 (segment (start 124.73 97.1) (end 124.73 101.94) (width 0.2) (layer "F.Cu") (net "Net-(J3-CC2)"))
 (segment (start 123.73 101.94) (end 123.73 97.42) (width 0.2) (layer "F.Cu") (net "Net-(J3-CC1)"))
 (segment (start 123.73 97.42) (end 122.65 96.34) (width 0.2) (layer "F.Cu") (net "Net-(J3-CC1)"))
 (segment (start 122.92 96.07) (end 122.65 96.34) (width 0.2) (layer "F.Cu") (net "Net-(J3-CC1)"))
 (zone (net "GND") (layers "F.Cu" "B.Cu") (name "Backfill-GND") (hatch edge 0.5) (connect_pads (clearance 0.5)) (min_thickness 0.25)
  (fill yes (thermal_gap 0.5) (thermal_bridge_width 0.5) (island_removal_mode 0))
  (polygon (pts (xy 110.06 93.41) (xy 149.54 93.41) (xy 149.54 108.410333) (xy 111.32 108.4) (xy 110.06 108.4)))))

